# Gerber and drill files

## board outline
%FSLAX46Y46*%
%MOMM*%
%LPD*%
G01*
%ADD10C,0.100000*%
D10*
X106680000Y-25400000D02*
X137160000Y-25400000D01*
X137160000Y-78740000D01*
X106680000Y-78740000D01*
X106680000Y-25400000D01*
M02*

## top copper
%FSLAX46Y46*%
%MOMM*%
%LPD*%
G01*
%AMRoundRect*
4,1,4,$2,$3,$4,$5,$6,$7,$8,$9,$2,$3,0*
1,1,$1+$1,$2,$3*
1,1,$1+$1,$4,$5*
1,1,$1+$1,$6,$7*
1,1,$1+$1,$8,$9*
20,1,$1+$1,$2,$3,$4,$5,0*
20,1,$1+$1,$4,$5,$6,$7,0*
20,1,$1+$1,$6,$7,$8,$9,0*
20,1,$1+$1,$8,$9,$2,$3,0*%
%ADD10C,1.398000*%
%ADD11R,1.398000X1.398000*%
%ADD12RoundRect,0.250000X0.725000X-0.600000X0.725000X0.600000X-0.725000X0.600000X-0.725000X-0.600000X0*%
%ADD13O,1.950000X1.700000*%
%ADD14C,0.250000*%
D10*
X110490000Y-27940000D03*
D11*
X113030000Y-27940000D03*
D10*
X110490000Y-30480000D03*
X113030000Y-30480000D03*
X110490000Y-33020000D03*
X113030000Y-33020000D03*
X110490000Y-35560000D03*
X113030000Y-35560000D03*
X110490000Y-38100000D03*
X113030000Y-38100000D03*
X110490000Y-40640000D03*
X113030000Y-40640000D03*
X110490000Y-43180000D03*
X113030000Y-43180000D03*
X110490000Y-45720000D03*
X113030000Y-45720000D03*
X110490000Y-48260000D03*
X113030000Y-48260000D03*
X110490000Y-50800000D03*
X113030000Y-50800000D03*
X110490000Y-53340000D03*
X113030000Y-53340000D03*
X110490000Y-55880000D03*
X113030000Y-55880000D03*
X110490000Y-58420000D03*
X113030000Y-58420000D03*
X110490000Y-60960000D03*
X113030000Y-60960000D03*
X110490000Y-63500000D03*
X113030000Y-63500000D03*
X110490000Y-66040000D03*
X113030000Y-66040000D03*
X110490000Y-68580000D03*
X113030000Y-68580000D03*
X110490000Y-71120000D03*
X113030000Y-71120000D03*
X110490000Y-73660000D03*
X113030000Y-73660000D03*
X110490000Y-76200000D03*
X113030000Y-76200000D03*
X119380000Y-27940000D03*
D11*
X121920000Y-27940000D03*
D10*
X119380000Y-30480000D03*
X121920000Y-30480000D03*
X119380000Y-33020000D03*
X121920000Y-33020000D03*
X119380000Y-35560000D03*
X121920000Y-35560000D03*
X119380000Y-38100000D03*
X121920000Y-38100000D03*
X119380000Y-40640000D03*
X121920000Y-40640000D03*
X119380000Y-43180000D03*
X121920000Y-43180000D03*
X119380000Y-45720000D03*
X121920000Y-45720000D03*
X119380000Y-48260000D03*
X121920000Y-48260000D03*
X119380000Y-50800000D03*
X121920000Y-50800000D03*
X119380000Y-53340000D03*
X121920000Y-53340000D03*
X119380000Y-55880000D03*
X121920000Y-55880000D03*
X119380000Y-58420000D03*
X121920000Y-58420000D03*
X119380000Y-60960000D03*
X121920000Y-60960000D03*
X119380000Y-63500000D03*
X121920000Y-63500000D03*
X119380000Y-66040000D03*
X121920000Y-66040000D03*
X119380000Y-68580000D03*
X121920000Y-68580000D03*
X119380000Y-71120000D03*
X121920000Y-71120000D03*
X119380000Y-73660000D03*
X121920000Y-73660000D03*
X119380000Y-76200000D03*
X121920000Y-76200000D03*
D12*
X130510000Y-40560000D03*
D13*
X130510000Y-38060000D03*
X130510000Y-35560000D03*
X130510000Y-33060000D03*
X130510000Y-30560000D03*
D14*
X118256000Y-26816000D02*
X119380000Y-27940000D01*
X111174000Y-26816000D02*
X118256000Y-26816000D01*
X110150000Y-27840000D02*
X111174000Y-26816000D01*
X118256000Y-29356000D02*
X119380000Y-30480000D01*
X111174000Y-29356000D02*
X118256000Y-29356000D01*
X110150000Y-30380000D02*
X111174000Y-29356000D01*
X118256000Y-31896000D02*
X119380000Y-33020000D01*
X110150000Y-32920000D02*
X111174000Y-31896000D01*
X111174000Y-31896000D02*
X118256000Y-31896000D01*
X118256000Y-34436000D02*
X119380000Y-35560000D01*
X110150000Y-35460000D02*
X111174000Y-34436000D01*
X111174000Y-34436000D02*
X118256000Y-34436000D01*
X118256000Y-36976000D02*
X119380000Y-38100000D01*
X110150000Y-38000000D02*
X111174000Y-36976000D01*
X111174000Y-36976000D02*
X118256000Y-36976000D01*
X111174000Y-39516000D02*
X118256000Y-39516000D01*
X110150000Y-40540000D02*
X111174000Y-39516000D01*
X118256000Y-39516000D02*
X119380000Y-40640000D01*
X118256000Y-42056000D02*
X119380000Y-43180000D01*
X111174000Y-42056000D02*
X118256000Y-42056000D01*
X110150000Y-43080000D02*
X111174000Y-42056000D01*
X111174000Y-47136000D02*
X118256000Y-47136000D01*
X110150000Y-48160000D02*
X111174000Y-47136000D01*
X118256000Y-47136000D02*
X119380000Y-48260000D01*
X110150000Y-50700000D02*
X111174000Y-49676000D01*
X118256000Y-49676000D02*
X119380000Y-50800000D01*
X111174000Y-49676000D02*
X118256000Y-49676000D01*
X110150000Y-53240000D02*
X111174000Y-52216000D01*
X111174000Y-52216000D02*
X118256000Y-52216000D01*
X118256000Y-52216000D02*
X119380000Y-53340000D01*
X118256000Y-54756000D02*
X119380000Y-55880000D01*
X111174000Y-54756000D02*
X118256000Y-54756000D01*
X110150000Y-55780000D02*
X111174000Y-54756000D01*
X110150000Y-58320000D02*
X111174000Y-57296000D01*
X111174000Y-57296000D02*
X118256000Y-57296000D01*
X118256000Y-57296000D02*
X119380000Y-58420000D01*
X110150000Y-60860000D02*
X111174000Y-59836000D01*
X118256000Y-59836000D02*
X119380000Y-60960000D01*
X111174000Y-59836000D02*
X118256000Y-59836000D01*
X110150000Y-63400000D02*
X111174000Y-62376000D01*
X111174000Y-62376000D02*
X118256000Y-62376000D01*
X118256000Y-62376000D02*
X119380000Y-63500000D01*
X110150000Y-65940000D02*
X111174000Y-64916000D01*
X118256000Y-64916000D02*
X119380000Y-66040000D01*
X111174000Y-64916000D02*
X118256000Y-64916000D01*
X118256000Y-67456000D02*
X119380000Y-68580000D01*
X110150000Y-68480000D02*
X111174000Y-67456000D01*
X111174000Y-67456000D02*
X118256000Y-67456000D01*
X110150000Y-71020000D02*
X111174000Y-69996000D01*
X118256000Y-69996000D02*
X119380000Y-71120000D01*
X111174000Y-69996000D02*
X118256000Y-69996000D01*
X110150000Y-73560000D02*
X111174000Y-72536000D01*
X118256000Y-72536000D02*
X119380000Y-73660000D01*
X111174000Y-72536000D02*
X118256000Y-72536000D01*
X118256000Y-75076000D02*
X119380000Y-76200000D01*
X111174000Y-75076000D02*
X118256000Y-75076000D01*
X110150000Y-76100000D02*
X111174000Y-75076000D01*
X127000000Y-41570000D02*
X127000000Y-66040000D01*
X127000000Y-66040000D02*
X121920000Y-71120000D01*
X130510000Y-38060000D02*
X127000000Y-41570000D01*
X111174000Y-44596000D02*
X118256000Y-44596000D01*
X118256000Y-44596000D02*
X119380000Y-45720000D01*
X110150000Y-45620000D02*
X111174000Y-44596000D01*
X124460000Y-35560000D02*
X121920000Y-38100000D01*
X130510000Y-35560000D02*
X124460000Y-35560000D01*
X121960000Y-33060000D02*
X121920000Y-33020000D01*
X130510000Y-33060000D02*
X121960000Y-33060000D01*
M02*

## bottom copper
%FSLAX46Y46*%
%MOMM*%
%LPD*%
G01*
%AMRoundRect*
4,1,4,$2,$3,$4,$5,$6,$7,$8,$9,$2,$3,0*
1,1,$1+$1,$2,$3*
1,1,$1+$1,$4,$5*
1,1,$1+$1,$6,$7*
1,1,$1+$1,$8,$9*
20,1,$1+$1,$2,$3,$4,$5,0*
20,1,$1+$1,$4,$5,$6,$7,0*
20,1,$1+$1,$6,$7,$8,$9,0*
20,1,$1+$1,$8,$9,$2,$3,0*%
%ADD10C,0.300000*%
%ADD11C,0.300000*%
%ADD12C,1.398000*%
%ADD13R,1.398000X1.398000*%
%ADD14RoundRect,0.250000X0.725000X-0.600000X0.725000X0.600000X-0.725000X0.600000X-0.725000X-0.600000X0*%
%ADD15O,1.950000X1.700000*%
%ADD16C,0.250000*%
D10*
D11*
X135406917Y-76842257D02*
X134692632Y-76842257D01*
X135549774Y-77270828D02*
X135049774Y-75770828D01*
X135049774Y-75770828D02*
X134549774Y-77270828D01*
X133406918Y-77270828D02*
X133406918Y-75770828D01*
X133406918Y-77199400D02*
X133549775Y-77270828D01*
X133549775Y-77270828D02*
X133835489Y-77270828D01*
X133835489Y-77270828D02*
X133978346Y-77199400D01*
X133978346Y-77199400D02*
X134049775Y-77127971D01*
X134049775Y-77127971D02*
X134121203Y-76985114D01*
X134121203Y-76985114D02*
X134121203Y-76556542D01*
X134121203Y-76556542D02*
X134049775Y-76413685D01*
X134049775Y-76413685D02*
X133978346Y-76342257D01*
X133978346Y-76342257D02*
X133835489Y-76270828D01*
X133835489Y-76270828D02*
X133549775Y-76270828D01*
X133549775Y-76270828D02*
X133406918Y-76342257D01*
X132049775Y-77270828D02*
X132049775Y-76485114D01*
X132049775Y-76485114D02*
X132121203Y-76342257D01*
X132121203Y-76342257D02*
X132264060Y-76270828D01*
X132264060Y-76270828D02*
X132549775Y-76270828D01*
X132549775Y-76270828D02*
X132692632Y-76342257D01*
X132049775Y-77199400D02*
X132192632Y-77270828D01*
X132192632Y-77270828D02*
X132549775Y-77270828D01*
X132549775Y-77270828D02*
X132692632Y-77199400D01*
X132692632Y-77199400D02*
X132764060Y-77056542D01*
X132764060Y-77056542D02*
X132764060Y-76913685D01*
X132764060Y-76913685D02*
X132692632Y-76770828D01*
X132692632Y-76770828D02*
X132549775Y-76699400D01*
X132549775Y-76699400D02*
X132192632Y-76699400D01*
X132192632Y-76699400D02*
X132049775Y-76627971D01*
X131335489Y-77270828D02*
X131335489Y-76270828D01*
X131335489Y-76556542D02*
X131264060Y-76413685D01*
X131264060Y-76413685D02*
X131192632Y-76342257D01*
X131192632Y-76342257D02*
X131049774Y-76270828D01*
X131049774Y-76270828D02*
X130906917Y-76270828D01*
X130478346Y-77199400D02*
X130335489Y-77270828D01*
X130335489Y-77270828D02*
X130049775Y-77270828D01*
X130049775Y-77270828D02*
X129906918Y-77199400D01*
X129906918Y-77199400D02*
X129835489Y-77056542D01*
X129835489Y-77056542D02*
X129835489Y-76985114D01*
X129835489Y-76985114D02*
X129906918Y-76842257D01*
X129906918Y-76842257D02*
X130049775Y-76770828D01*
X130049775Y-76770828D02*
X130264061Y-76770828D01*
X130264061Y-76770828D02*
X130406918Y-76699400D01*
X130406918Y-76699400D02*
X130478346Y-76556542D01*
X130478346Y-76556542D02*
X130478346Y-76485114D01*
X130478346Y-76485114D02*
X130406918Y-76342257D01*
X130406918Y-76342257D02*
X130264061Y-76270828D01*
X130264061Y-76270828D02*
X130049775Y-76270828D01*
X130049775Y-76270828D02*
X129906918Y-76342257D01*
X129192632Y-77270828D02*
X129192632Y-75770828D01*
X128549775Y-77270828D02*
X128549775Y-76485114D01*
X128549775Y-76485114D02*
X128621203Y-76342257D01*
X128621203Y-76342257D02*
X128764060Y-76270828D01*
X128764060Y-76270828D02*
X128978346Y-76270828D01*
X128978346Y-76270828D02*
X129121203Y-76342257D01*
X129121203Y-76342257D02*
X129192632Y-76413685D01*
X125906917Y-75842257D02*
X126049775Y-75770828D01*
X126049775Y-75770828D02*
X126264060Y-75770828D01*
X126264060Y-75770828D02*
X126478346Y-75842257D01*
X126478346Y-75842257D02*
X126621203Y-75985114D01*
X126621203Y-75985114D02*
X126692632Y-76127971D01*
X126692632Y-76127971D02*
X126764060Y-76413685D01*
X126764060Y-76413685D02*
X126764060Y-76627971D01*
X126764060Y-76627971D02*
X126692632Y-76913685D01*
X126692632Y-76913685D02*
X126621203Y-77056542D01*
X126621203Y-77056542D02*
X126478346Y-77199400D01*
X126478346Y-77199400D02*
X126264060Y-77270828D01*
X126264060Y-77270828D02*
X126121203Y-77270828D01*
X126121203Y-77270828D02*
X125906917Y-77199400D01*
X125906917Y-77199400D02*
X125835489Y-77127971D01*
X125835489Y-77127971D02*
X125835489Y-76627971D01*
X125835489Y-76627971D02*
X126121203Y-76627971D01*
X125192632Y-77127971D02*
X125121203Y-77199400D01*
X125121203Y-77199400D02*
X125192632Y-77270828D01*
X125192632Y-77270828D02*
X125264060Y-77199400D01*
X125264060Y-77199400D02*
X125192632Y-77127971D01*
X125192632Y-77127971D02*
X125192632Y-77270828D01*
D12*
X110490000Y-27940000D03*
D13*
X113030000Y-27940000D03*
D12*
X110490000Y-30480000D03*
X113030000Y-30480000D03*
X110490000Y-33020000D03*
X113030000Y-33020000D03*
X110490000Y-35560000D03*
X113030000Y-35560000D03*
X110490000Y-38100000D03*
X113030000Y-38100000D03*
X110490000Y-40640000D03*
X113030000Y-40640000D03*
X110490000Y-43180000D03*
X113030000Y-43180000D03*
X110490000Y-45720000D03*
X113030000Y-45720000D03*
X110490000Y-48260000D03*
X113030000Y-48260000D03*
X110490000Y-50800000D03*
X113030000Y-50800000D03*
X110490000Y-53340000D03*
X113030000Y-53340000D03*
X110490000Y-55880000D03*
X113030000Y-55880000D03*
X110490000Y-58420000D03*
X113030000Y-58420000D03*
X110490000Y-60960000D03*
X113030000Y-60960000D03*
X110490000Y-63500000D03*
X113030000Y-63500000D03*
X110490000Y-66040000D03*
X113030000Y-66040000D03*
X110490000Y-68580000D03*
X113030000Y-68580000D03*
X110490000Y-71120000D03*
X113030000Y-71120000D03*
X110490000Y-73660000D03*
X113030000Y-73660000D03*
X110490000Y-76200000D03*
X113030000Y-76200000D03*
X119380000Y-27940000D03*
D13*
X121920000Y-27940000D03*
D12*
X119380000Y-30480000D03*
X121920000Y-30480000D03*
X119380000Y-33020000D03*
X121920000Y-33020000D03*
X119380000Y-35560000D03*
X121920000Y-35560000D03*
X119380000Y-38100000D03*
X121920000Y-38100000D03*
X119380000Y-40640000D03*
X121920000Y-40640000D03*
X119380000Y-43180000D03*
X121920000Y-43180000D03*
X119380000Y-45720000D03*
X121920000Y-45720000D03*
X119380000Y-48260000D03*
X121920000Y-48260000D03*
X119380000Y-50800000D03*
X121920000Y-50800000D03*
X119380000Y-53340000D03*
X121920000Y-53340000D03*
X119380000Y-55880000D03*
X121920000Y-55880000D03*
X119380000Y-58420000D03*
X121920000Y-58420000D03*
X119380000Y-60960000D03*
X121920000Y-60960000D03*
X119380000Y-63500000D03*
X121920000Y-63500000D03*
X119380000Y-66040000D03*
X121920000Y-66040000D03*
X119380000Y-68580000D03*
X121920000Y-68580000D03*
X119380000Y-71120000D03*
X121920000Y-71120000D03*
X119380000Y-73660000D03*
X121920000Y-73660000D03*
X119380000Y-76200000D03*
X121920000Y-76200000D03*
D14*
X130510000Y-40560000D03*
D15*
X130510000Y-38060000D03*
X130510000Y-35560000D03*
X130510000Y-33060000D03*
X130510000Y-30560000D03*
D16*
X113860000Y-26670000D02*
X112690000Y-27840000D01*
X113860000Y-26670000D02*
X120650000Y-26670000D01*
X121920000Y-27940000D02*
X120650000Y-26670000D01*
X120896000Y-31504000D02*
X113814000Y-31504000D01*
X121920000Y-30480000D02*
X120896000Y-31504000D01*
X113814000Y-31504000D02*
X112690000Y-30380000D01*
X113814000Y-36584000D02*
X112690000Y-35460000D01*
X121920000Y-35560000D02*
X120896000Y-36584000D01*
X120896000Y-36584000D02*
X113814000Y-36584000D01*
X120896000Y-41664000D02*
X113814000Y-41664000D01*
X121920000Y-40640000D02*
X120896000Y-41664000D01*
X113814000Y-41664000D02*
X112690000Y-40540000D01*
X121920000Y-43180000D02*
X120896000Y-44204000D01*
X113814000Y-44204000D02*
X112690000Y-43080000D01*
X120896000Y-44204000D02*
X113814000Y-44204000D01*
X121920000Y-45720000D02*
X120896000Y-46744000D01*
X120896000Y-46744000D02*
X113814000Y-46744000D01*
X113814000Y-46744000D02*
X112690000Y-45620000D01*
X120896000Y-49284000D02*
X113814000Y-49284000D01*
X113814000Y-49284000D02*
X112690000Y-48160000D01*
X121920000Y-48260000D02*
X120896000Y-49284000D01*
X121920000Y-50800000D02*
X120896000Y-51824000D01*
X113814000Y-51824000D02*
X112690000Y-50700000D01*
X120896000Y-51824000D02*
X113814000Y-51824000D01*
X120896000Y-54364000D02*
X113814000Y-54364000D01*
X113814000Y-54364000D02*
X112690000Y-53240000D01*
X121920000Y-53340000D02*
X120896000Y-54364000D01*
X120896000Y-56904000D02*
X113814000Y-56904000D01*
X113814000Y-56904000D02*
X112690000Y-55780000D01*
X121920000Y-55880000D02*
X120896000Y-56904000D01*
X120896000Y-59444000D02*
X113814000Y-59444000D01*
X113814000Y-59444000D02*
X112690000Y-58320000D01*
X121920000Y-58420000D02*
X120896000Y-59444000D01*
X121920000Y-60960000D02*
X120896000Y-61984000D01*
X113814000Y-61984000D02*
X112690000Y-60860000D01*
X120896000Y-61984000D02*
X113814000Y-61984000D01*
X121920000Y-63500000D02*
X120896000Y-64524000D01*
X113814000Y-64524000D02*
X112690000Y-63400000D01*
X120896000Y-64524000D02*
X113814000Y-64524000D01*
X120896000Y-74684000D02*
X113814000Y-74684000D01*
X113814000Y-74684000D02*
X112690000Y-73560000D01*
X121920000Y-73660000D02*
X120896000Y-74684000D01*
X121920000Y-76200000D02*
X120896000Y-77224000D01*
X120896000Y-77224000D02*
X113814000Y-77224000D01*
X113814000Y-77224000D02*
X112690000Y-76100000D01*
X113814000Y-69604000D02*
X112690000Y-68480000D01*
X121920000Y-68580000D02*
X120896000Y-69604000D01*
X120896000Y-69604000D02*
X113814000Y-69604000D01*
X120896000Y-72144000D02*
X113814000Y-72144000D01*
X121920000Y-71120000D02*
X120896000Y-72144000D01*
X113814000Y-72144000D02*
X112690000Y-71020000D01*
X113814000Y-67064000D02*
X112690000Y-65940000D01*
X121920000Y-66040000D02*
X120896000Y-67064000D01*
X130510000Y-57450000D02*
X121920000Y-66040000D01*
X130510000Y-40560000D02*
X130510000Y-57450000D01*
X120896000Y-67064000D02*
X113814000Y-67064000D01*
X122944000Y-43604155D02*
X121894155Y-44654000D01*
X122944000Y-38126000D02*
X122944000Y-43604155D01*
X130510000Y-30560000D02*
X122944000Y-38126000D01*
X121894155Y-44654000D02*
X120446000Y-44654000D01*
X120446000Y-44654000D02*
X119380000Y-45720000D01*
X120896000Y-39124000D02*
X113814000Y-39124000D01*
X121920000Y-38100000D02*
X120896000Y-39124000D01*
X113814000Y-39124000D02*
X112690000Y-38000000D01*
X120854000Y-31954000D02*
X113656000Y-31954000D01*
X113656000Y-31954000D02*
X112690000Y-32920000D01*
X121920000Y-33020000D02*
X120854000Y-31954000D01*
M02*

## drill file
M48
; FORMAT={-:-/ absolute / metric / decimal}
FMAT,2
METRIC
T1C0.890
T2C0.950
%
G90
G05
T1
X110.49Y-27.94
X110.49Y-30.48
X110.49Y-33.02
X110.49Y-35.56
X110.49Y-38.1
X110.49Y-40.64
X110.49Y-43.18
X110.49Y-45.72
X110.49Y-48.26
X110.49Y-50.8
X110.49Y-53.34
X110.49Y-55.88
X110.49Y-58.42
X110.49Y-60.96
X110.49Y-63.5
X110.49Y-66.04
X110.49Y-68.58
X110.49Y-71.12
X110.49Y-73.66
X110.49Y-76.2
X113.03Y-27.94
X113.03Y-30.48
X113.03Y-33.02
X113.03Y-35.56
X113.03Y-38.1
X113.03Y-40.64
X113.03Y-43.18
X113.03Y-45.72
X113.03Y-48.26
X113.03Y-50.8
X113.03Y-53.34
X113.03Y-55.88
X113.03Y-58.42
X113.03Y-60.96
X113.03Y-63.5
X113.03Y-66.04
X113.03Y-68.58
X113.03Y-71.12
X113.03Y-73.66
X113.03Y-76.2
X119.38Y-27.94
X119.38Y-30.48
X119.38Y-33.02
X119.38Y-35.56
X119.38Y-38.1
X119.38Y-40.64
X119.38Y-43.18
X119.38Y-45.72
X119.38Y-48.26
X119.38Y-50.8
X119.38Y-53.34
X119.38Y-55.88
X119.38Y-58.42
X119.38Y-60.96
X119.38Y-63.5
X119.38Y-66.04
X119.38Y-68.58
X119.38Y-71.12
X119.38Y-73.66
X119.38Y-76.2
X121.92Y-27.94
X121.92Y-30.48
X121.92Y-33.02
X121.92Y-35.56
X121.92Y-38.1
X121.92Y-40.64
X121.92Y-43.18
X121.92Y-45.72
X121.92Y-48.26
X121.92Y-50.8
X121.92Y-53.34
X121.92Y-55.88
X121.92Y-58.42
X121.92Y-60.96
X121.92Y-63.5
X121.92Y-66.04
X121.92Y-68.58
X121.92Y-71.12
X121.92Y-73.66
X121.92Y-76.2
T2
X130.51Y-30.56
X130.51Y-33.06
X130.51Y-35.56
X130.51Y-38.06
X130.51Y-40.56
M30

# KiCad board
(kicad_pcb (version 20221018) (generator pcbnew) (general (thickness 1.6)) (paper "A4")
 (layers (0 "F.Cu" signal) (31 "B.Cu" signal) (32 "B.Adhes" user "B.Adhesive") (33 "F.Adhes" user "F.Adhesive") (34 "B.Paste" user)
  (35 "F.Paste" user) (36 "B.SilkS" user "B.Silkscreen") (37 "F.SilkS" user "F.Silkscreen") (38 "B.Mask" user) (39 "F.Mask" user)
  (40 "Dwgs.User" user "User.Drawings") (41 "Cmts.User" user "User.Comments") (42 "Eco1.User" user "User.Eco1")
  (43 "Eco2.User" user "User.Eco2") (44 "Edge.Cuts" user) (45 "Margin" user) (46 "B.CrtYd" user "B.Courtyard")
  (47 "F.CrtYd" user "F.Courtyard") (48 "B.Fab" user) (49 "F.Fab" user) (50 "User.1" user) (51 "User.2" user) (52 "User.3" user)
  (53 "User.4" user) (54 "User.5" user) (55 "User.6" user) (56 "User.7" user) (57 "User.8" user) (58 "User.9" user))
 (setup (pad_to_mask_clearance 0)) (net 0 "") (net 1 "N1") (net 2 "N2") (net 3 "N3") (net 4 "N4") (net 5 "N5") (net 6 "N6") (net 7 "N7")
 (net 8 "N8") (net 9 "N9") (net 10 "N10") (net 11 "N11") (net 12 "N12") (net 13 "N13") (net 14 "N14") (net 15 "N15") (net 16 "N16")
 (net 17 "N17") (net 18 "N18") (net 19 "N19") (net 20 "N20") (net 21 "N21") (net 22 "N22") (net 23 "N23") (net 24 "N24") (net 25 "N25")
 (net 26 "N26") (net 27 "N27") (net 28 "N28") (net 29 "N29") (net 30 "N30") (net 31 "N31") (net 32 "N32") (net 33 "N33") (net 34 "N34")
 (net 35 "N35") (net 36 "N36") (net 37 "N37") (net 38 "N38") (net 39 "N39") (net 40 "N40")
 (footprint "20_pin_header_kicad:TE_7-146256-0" (layer "F.Cu") (at 111.76 52.07 -90)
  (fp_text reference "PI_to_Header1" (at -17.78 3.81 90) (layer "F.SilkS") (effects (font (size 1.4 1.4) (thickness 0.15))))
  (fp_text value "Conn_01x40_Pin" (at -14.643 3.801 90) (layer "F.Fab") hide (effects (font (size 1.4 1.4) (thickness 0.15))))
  (pad "1" thru_hole circle (at -24.13 1.27 270) (size 1.398 1.398) (drill 0.89) (layers "*.Cu" "*.Mask") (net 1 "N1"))
  (pad "2" thru_hole rect (at -24.13 -1.27 270) (size 1.398 1.398) (drill 0.89) (layers "*.Cu" "*.Mask") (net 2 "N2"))
  (pad "3" thru_hole circle (at -21.59 1.27 270) (size 1.398 1.398) (drill 0.89) (layers "*.Cu" "*.Mask") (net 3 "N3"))
  (pad "4" thru_hole circle (at -21.59 -1.27 270) (size 1.398 1.398) (drill 0.89) (layers "*.Cu" "*.Mask") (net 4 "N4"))
  (pad "5" thru_hole circle (at -19.05 1.27 270) (size 1.398 1.398) (drill 0.89) (layers "*.Cu" "*.Mask") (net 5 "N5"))
  (pad "6" thru_hole circle (at -19.05 -1.27 270) (size 1.398 1.398) (drill 0.89) (layers "*.Cu" "*.Mask") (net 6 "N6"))
  (pad "7" thru_hole circle (at -16.51 1.27 270) (size 1.398 1.398) (drill 0.89) (layers "*.Cu" "*.Mask") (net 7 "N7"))
  (pad "8" thru_hole circle (at -16.51 -1.27 270) (size 1.398 1.398) (drill 0.89) (layers "*.Cu" "*.Mask") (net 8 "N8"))
  (pad "9" thru_hole circle (at -13.97 1.27 270) (size 1.398 1.398) (drill 0.89) (layers "*.Cu" "*.Mask") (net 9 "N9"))
  (pad "10" thru_hole circle (at -13.97 -1.27 270) (size 1.398 1.398) (drill 0.89) (layers "*.Cu" "*.Mask") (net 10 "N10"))
  (pad "11" thru_hole circle (at -11.43 1.27 270) (size 1.398 1.398) (drill 0.89) (layers "*.Cu" "*.Mask") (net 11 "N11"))
  (pad "12" thru_hole circle (at -11.43 -1.27 270) (size 1.398 1.398) (drill 0.89) (layers "*.Cu" "*.Mask") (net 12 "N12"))
  (pad "13" thru_hole circle (at -8.89 1.27 270) (size 1.398 1.398) (drill 0.89) (layers "*.Cu" "*.Mask") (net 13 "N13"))
  (pad "14" thru_hole circle (at -8.89 -1.27 270) (size 1.398 1.398) (drill 0.89) (layers "*.Cu" "*.Mask") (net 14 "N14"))
  (pad "15" thru_hole circle (at -6.35 1.27 270) (size 1.398 1.398) (drill 0.89) (layers "*.Cu" "*.Mask") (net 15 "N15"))
  (pad "16" thru_hole circle (at -6.35 -1.27 270) (size 1.398 1.398) (drill 0.89) (layers "*.Cu" "*.Mask") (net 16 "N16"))
  (pad "17" thru_hole circle (at -3.81 1.27 270) (size 1.398 1.398) (drill 0.89) (layers "*.Cu" "*.Mask") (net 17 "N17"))
  (pad "18" thru_hole circle (at -3.81 -1.27 270) (size 1.398 1.398) (drill 0.89) (layers "*.Cu" "*.Mask") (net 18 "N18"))
  (pad "19" thru_hole circle (at -1.27 1.27 270) (size 1.398 1.398) (drill 0.89) (layers "*.Cu" "*.Mask") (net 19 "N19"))
  (pad "20" thru_hole circle (at -1.27 -1.27 270) (size 1.398 1.398) (drill 0.89) (layers "*.Cu" "*.Mask") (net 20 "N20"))
  (pad "21" thru_hole circle (at 1.27 1.27 270) (size 1.398 1.398) (drill 0.89) (layers "*.Cu" "*.Mask") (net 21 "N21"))
  (pad "22" thru_hole circle (at 1.27 -1.27 270) (size 1.398 1.398) (drill 0.89) (layers "*.Cu" "*.Mask") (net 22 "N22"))
  (pad "23" thru_hole circle (at 3.81 1.27 270) (size 1.398 1.398) (drill 0.89) (layers "*.Cu" "*.Mask") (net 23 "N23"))
  (pad "24" thru_hole circle (at 3.81 -1.27 270) (size 1.398 1.398) (drill 0.89) (layers "*.Cu" "*.Mask") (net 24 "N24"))
  (pad "25" thru_hole circle (at 6.35 1.27 270) (size 1.398 1.398) (drill 0.89) (layers "*.Cu" "*.Mask") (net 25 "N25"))
  (pad "26" thru_hole circle (at 6.35 -1.27 270) (size 1.398 1.398) (drill 0.89) (layers "*.Cu" "*.Mask") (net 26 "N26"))
  (pad "27" thru_hole circle (at 8.89 1.27 270) (size 1.398 1.398) (drill 0.89) (layers "*.Cu" "*.Mask") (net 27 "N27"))
  (pad "28" thru_hole circle (at 8.89 -1.27 270) (size 1.398 1.398) (drill 0.89) (layers "*.Cu" "*.Mask") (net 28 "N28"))
  (pad "29" thru_hole circle (at 11.43 1.27 270) (size 1.398 1.398) (drill 0.89) (layers "*.Cu" "*.Mask") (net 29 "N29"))
  (pad "30" thru_hole circle (at 11.43 -1.27 270) (size 1.398 1.398) (drill 0.89) (layers "*.Cu" "*.Mask") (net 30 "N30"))
  (pad "31" thru_hole circle (at 13.97 1.27 270) (size 1.398 1.398) (drill 0.89) (layers "*.Cu" "*.Mask") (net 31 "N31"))
  (pad "32" thru_hole circle (at 13.97 -1.27 270) (size 1.398 1.398) (drill 0.89) (layers "*.Cu" "*.Mask") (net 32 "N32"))
  (pad "33" thru_hole circle (at 16.51 1.27 270) (size 1.398 1.398) (drill 0.89) (layers "*.Cu" "*.Mask") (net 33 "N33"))
  (pad "34" thru_hole circle (at 16.51 -1.27 270) (size 1.398 1.398) (drill 0.89) (layers "*.Cu" "*.Mask") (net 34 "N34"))
  (pad "35" thru_hole circle (at 19.05 1.27 270) (size 1.398 1.398) (drill 0.89) (layers "*.Cu" "*.Mask") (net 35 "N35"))
  (pad "36" thru_hole circle (at 19.05 -1.27 270) (size 1.398 1.398) (drill 0.89) (layers "*.Cu" "*.Mask") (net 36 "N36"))
  (pad "37" thru_hole circle (at 21.59 1.27 270) (size 1.398 1.398) (drill 0.89) (layers "*.Cu" "*.Mask") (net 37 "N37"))
  (pad "38" thru_hole circle (at 21.59 -1.27 270) (size 1.398 1.398) (drill 0.89) (layers "*.Cu" "*.Mask") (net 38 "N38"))
  (pad "39" thru_hole circle (at 24.13 1.27 270) (size 1.398 1.398) (drill 0.89) (layers "*.Cu" "*.Mask") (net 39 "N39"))
  (pad "40" thru_hole circle (at 24.13 -1.27 270) (size 1.398 1.398) (drill 0.89) (layers "*.Cu" "*.Mask") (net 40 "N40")))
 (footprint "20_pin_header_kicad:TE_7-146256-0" (layer "F.Cu") (at 120.65 52.07 -90)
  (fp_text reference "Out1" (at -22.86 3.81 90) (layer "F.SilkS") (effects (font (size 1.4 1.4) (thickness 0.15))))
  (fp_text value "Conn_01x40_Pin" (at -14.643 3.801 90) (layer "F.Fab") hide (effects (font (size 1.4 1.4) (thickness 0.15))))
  (pad "1" thru_hole circle (at -24.13 1.27 270) (size 1.398 1.398) (drill 0.89) (layers "*.Cu" "*.Mask") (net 1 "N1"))
  (pad "2" thru_hole rect (at -24.13 -1.27 270) (size 1.398 1.398) (drill 0.89) (layers "*.Cu" "*.Mask") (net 2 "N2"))
  (pad "3" thru_hole circle (at -21.59 1.27 270) (size 1.398 1.398) (drill 0.89) (layers "*.Cu" "*.Mask") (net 3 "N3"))
  (pad "4" thru_hole circle (at -21.59 -1.27 270) (size 1.398 1.398) (drill 0.89) (layers "*.Cu" "*.Mask") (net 4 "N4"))
  (pad "5" thru_hole circle (at -19.05 1.27 270) (size 1.398 1.398) (drill 0.89) (layers "*.Cu" "*.Mask") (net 5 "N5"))
  (pad "6" thru_hole circle (at -19.05 -1.27 270) (size 1.398 1.398) (drill 0.89) (layers "*.Cu" "*.Mask") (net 6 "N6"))
  (pad "7" thru_hole circle (at -16.51 1.27 270) (size 1.398 1.398) (drill 0.89) (layers "*.Cu" "*.Mask") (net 7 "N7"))
  (pad "8" thru_hole circle (at -16.51 -1.27 270) (size 1.398 1.398) (drill 0.89) (layers "*.Cu" "*.Mask") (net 8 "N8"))
  (pad "9" thru_hole circle (at -13.97 1.27 270) (size 1.398 1.398) (drill 0.89) (layers "*.Cu" "*.Mask") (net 9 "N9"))
  (pad "10" thru_hole circle (at -13.97 -1.27 270) (size 1.398 1.398) (drill 0.89) (layers "*.Cu" "*.Mask") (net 10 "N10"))
  (pad "11" thru_hole circle (at -11.43 1.27 270) (size 1.398 1.398) (drill 0.89) (layers "*.Cu" "*.Mask") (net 11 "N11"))
  (pad "12" thru_hole circle (at -11.43 -1.27 270) (size 1.398 1.398) (drill 0.89) (layers "*.Cu" "*.Mask") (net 12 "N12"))
  (pad "13" thru_hole circle (at -8.89 1.27 270) (size 1.398 1.398) (drill 0.89) (layers "*.Cu" "*.Mask") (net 13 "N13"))
  (pad "14" thru_hole circle (at -8.89 -1.27 270) (size 1.398 1.398) (drill 0.89) (layers "*.Cu" "*.Mask") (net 14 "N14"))
  (pad "15" thru_hole circle (at -6.35 1.27 270) (size 1.398 1.398) (drill 0.89) (layers "*.Cu" "*.Mask") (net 15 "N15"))
  (pad "16" thru_hole circle (at -6.35 -1.27 270) (size 1.398 1.398) (drill 0.89) (layers "*.Cu" "*.Mask") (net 16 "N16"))
  (pad "17" thru_hole circle (at -3.81 1.27 270) (size 1.398 1.398) (drill 0.89) (layers "*.Cu" "*.Mask") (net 17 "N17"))
  (pad "18" thru_hole circle (at -3.81 -1.27 270) (size 1.398 1.398) (drill 0.89) (layers "*.Cu" "*.Mask") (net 18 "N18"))
  (pad "19" thru_hole circle (at -1.27 1.27 270) (size 1.398 1.398) (drill 0.89) (layers "*.Cu" "*.Mask") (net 19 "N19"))
  (pad "20" thru_hole circle (at -1.27 -1.27 270) (size 1.398 1.398) (drill 0.89) (layers "*.Cu" "*.Mask") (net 20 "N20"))
  (pad "21" thru_hole circle (at 1.27 1.27 270) (size 1.398 1.398) (drill 0.89) (layers "*.Cu" "*.Mask") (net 21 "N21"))
  (pad "22" thru_hole circle (at 1.27 -1.27 270) (size 1.398 1.398) (drill 0.89) (layers "*.Cu" "*.Mask") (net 22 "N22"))
  (pad "23" thru_hole circle (at 3.81 1.27 270) (size 1.398 1.398) (drill 0.89) (layers "*.Cu" "*.Mask") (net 23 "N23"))
  (pad "24" thru_hole circle (at 3.81 -1.27 270) (size 1.398 1.398) (drill 0.89) (layers "*.Cu" "*.Mask") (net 24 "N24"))
  (pad "25" thru_hole circle (at 6.35 1.27 270) (size 1.398 1.398) (drill 0.89) (layers "*.Cu" "*.Mask") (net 25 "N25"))
  (pad "26" thru_hole circle (at 6.35 -1.27 270) (size 1.398 1.398) (drill 0.89) (layers "*.Cu" "*.Mask") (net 26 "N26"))
  (pad "27" thru_hole circle (at 8.89 1.27 270) (size 1.398 1.398) (drill 0.89) (layers "*.Cu" "*.Mask") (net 27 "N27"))
  (pad "28" thru_hole circle (at 8.89 -1.27 270) (size 1.398 1.398) (drill 0.89) (layers "*.Cu" "*.Mask") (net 28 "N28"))
  (pad "29" thru_hole circle (at 11.43 1.27 270) (size 1.398 1.398) (drill 0.89) (layers "*.Cu" "*.Mask") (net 29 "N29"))
  (pad "30" thru_hole circle (at 11.43 -1.27 270) (size 1.398 1.398) (drill 0.89) (layers "*.Cu" "*.Mask") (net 30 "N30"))
  (pad "31" thru_hole circle (at 13.97 1.27 270) (size 1.398 1.398) (drill 0.89) (layers "*.Cu" "*.Mask") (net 31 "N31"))
  (pad "32" thru_hole circle (at 13.97 -1.27 270) (size 1.398 1.398) (drill 0.89) (layers "*.Cu" "*.Mask") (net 32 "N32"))
  (pad "33" thru_hole circle (at 16.51 1.27 270) (size 1.398 1.398) (drill 0.89) (layers "*.Cu" "*.Mask") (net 33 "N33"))
  (pad "34" thru_hole circle (at 16.51 -1.27 270) (size 1.398 1.398) (drill 0.89) (layers "*.Cu" "*.Mask") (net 34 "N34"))
  (pad "35" thru_hole circle (at 19.05 1.27 270) (size 1.398 1.398) (drill 0.89) (layers "*.Cu" "*.Mask") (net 35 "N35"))
  (pad "36" thru_hole circle (at 19.05 -1.27 270) (size 1.398 1.398) (drill 0.89) (layers "*.Cu" "*.Mask") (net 36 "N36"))
  (pad "37" thru_hole circle (at 21.59 1.27 270) (size 1.398 1.398) (drill 0.89) (layers "*.Cu" "*.Mask") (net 37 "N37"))
  (pad "38" thru_hole circle (at 21.59 -1.27 270) (size 1.398 1.398) (drill 0.89) (layers "*.Cu" "*.Mask") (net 38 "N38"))
  (pad "39" thru_hole circle (at 24.13 1.27 270) (size 1.398 1.398) (drill 0.89) (layers "*.Cu" "*.Mask") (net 39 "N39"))
  (pad "40" thru_hole circle (at 24.13 -1.27 270) (size 1.398 1.398) (drill 0.89) (layers "*.Cu" "*.Mask") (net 40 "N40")))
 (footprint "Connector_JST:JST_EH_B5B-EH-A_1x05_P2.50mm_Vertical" (layer "F.Cu") (at 130.51 40.56 90)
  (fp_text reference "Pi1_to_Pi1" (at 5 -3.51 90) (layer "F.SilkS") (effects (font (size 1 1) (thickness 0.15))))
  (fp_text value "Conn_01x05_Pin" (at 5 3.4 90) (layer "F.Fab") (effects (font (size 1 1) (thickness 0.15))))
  (pad "1" thru_hole roundrect (at 0 0 90) (size 1.7 1.95) (drill 0.95) (layers "*.Cu" "*.Mask") (roundrect_rratio 0.1470588235)
   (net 32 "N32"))
  (pad "2" thru_hole oval (at 2.5 0 90) (size 1.7 1.95) (drill 0.95) (layers "*.Cu" "*.Mask") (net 36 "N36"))
  (pad "3" thru_hole oval (at 5 0 90) (size 1.7 1.95) (drill 0.95) (layers "*.Cu" "*.Mask") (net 10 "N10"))
  (pad "4" thru_hole oval (at 7.5 0 90) (size 1.7 1.95) (drill 0.95) (layers "*.Cu" "*.Mask") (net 6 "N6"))
  (pad "5" thru_hole oval (at 10 0 90) (size 1.7 1.95) (drill 0.95) (layers "*.Cu" "*.Mask") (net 15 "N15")))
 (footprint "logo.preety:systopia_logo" (layer "F.Cu") (at 130.81 68.58)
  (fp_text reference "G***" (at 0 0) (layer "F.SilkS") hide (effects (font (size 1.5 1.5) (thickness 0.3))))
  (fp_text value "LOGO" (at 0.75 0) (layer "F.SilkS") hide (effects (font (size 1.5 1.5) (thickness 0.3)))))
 (gr_rect (start 106.68 25.4) (end 137.16 78.74) (stroke (width 0.1) (type default)) (fill none) (layer "Edge.Cuts"))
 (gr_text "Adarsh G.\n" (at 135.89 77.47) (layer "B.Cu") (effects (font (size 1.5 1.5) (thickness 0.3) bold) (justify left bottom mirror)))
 (segment (start 118.256 26.816) (end 119.38 27.94) (width 0.25) (layer "F.Cu") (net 1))
 (segment (start 111.174 26.816) (end 118.256 26.816) (width 0.25) (layer "F.Cu") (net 1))
 (segment (start 110.15 27.84) (end 111.174 26.816) (width 0.25) (layer "F.Cu") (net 1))
 (segment (start 113.86 26.67) (end 112.69 27.84) (width 0.25) (layer "B.Cu") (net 2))
 (segment (start 113.86 26.67) (end 120.65 26.67) (width 0.25) (layer "B.Cu") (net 2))
 (segment (start 121.92 27.94) (end 120.65 26.67) (width 0.25) (layer "B.Cu") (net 2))
 (segment (start 118.256 29.356) (end 119.38 30.48) (width 0.25) (layer "F.Cu") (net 3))
 (segment (start 111.174 29.356) (end 118.256 29.356) (width 0.25) (layer "F.Cu") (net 3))
 (segment (start 110.15 30.38) (end 111.174 29.356) (width 0.25) (layer "F.Cu") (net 3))
 (segment (start 120.896 31.504) (end 113.814 31.504) (width 0.25) (layer "B.Cu") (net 4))
 (segment (start 121.92 30.48) (end 120.896 31.504) (width 0.25) (layer "B.Cu") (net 4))
 (segment (start 113.814 31.504) (end 112.69 30.38) (width 0.25) (layer "B.Cu") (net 4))
 (segment (start 118.256 31.896) (end 119.38 33.02) (width 0.25) (layer "F.Cu") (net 5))
 (segment (start 110.15 32.92) (end 111.174 31.896) (width 0.25) (layer "F.Cu") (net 5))
 (segment (start 111.174 31.896) (end 118.256 31.896) (width 0.25) (layer "F.Cu") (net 5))
 (segment (start 118.256 34.436) (end 119.38 35.56) (width 0.25) (layer "F.Cu") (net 7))
 (segment (start 110.15 35.46) (end 111.174 34.436) (width 0.25) (layer "F.Cu") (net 7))
 (segment (start 111.174 34.436) (end 118.256 34.436) (width 0.25) (layer "F.Cu") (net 7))
 (segment (start 113.814 36.584) (end 112.69 35.46) (width 0.25) (layer "B.Cu") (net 8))
 (segment (start 121.92 35.56) (end 120.896 36.584) (width 0.25) (layer "B.Cu") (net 8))
 (segment (start 120.896 36.584) (end 113.814 36.584) (width 0.25) (layer "B.Cu") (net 8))
 (segment (start 118.256 36.976) (end 119.38 38.1) (width 0.25) (layer "F.Cu") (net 9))
 (segment (start 110.15 38) (end 111.174 36.976) (width 0.25) (layer "F.Cu") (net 9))
 (segment (start 111.174 36.976) (end 118.256 36.976) (width 0.25) (layer "F.Cu") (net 9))
 (segment (start 111.174 39.516) (end 118.256 39.516) (width 0.25) (layer "F.Cu") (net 11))
 (segment (start 110.15 40.54) (end 111.174 39.516) (width 0.25) (layer "F.Cu") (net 11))
 (segment (start 118.256 39.516) (end 119.38 40.64) (width 0.25) (layer "F.Cu") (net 11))
 (segment (start 120.896 41.664) (end 113.814 41.664) (width 0.25) (layer "B.Cu") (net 12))
 (segment (start 121.92 40.64) (end 120.896 41.664) (width 0.25) (layer "B.Cu") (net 12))
 (segment (start 113.814 41.664) (end 112.69 40.54) (width 0.25) (layer "B.Cu") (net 12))
 (segment (start 118.256 42.056) (end 119.38 43.18) (width 0.25) (layer "F.Cu") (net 13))
 (segment (start 111.174 42.056) (end 118.256 42.056) (width 0.25) (layer "F.Cu") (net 13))
 (segment (start 110.15 43.08) (end 111.174 42.056) (width 0.25) (layer "F.Cu") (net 13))
 (segment (start 121.92 43.18) (end 120.896 44.204) (width 0.25) (layer "B.Cu") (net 14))
 (segment (start 113.814 44.204) (end 112.69 43.08) (width 0.25) (layer "B.Cu") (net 14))
 (segment (start 120.896 44.204) (end 113.814 44.204) (width 0.25) (layer "B.Cu") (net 14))
 (segment (start 121.92 45.72) (end 120.896 46.744) (width 0.25) (layer "B.Cu") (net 16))
 (segment (start 120.896 46.744) (end 113.814 46.744) (width 0.25) (layer "B.Cu") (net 16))
 (segment (start 113.814 46.744) (end 112.69 45.62) (width 0.25) (layer "B.Cu") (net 16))
 (segment (start 111.174 47.136) (end 118.256 47.136) (width 0.25) (layer "F.Cu") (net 17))
 (segment (start 110.15 48.16) (end 111.174 47.136) (width 0.25) (layer "F.Cu") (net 17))
 (segment (start 118.256 47.136) (end 119.38 48.26) (width 0.25) (layer "F.Cu") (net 17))
 (segment (start 120.896 49.284) (end 113.814 49.284) (width 0.25) (layer "B.Cu") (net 18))
 (segment (start 113.814 49.284) (end 112.69 48.16) (width 0.25) (layer "B.Cu") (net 18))
 (segment (start 121.92 48.26) (end 120.896 49.284) (width 0.25) (layer "B.Cu") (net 18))
 (segment (start 110.15 50.7) (end 111.174 49.676) (width 0.25) (layer "F.Cu") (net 19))
 (segment (start 118.256 49.676) (end 119.38 50.8) (width 0.25) (layer "F.Cu") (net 19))
 (segment (start 111.174 49.676) (end 118.256 49.676) (width 0.25) (layer "F.Cu") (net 19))
 (segment (start 121.92 50.8) (end 120.896 51.824) (width 0.25) (layer "B.Cu") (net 20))
 (segment (start 113.814 51.824) (end 112.69 50.7) (width 0.25) (layer "B.Cu") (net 20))
 (segment (start 120.896 51.824) (end 113.814 51.824) (width 0.25) (layer "B.Cu") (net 20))
 (segment (start 110.15 53.24) (end 111.174 52.216) (width 0.25) (layer "F.Cu") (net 21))
 (segment (start 111.174 52.216) (end 118.256 52.216) (width 0.25) (layer "F.Cu") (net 21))
 (segment (start 118.256 52.216) (end 119.38 53.34) (width 0.25) (layer "F.Cu") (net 21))
 (segment (start 120.896 54.364) (end 113.814 54.364) (width 0.25) (layer "B.Cu") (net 22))
 (segment (start 113.814 54.364) (end 112.69 53.24) (width 0.25) (layer "B.Cu") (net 22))
 (segment (start 121.92 53.34) (end 120.896 54.364) (width 0.25) (layer "B.Cu") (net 22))
 (segment (start 118.256 54.756) (end 119.38 55.88) (width 0.25) (layer "F.Cu") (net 23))
 (segment (start 111.174 54.756) (end 118.256 54.756) (width 0.25) (layer "F.Cu") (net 23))
 (segment (start 110.15 55.78) (end 111.174 54.756) (width 0.25) (layer "F.Cu") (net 23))
 (segment (start 120.896 56.904) (end 113.814 56.904) (width 0.25) (layer "B.Cu") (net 24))
 (segment (start 113.814 56.904) (end 112.69 55.78) (width 0.25) (layer "B.Cu") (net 24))
 (segment (start 121.92 55.88) (end 120.896 56.904) (width 0.25) (layer "B.Cu") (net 24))
 (segment (start 110.15 58.32) (end 111.174 57.296) (width 0.25) (layer "F.Cu") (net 25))
 (segment (start 111.174 57.296) (end 118.256 57.296) (width 0.25) (layer "F.Cu") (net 25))
 (segment (start 118.256 57.296) (end 119.38 58.42) (width 0.25) (layer "F.Cu") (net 25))
 (segment (start 120.896 59.444) (end 113.814 59.444) (width 0.25) (layer "B.Cu") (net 26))
 (segment (start 113.814 59.444) (end 112.69 58.32) (width 0.25) (layer "B.Cu") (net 26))
 (segment (start 121.92 58.42) (end 120.896 59.444) (width 0.25) (layer "B.Cu") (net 26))
 (segment (start 110.15 60.86) (end 111.174 59.836) (width 0.25) (layer "F.Cu") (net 27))
 (segment (start 118.256 59.836) (end 119.38 60.96) (width 0.25) (layer "F.Cu") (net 27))
 (segment (start 111.174 59.836) (end 118.256 59.836) (width 0.25) (layer "F.Cu") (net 27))
 (segment (start 121.92 60.96) (end 120.896 61.984) (width 0.25) (layer "B.Cu") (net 28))
 (segment (start 113.814 61.984) (end 112.69 60.86) (width 0.25) (layer "B.Cu") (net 28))
 (segment (start 120.896 61.984) (end 113.814 61.984) (width 0.25) (layer "B.Cu") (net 28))
 (segment (start 110.15 63.4) (end 111.174 62.376) (width 0.25) (layer "F.Cu") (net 29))
 (segment (start 111.174 62.376) (end 118.256 62.376) (width 0.25) (layer "F.Cu") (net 29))
 (segment (start 118.256 62.376) (end 119.38 63.5) (width 0.25) (layer "F.Cu") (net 29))
 (segment (start 121.92 63.5) (end 120.896 64.524) (width 0.25) (layer "B.Cu") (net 30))
 (segment (start 113.814 64.524) (end 112.69 63.4) (width 0.25) (layer "B.Cu") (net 30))
 (segment (start 120.896 64.524) (end 113.814 64.524) (width 0.25) (layer "B.Cu") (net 30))
 (segment (start 110.15 65.94) (end 111.174 64.916) (width 0.25) (layer "F.Cu") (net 31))
 (segment (start 118.256 64.916) (end 119.38 66.04) (width 0.25) (layer "F.Cu") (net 31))
 (segment (start 111.174 64.916) (end 118.256 64.916) (width 0.25) (layer "F.Cu") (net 31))
 (segment (start 118.256 67.456) (end 119.38 68.58) (width 0.25) (layer "F.Cu") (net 33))
 (segment (start 110.15 68.48) (end 111.174 67.456) (width 0.25) (layer "F.Cu") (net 33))
 (segment (start 111.174 67.456) (end 118.256 67.456) (width 0.25) (layer "F.Cu") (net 33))
 (segment (start 110.15 71.02) (end 111.174 69.996) (width 0.25) (layer "F.Cu") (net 35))
 (segment (start 118.256 69.996) (end 119.38 71.12) (width 0.25) (layer "F.Cu") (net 35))
 (segment (start 111.174 69.996) (end 118.256 69.996) (width 0.25) (layer "F.Cu") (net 35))
 (segment (start 110.15 73.56) (end 111.174 72.536) (width 0.25) (layer "F.Cu") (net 37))
 (segment (start 118.256 72.536) (end 119.38 73.66) (width 0.25) (layer "F.Cu") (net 37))
 (segment (start 111.174 72.536) (end 118.256 72.536) (width 0.25) (layer "F.Cu") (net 37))
 (segment (start 120.896 74.684) (end 113.814 74.684) (width 0.25) (layer "B.Cu") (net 38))
 (segment (start 113.814 74.684) (end 112.69 73.56) (width 0.25) (layer "B.Cu") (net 38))
 (segment (start 121.92 73.66) (end 120.896 74.684) (width 0.25) (layer "B.Cu") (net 38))
 (segment (start 118.256 75.076) (end 119.38 76.2) (width 0.25) (layer "F.Cu") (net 39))
 (segment (start 111.174 75.076) (end 118.256 75.076) (width 0.25) (layer "F.Cu") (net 39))
 (segment (start 110.15 76.1) (end 111.174 75.076) (width 0.25) (layer "F.Cu") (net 39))
 (segment (start 121.92 76.2) (end 120.896 77.224) (width 0.25) (layer "B.Cu") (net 40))
 (segment (start 120.896 77.224) (end 113.814 77.224) (width 0.25) (layer "B.Cu") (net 40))
 (segment (start 113.814 77.224) (end 112.69 76.1) (width 0.25) (layer "B.Cu") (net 40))
 (segment (start 113.814 69.604) (end 112.69 68.48) (width 0.25) (layer "B.Cu") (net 34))
 (segment (start 121.92 68.58) (end 120.896 69.604) (width 0.25) (layer "B.Cu") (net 34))
 (segment (start 120.896 69.604) (end 113.814 69.604) (width 0.25) (layer "B.Cu") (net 34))
 (segment (start 127 41.57) (end 127 66.04) (width 0.25) (layer "F.Cu") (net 36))
 (segment (start 127 66.04) (end 121.92 71.12) (width 0.25) (layer "F.Cu") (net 36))
 (segment (start 130.51 38.06) (end 127 41.57) (width 0.25) (layer "F.Cu") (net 36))
 (segment (start 120.896 72.144) (end 113.814 72.144) (width 0.25) (layer "B.Cu") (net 36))
 (segment (start 121.92 71.12) (end 120.896 72.144) (width 0.25) (layer "B.Cu") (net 36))
 (segment (start 113.814 72.144) (end 112.69 71.02) (width 0.25) (layer "B.Cu") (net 36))
 (segment (start 113.814 67.064) (end 112.69 65.94) (width 0.25) (layer "B.Cu") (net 32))
 (segment (start 121.92 66.04) (end 120.896 67.064) (width 0.25) (layer "B.Cu") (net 32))
 (segment (start 130.51 57.45) (end 121.92 66.04) (width 0.25) (layer "B.Cu") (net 32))
 (segment (start 130.51 40.56) (end 130.51 57.45) (width 0.25) (layer "B.Cu") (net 32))
 (segment (start 120.896 67.064) (end 113.814 67.064) (width 0.25) (layer "B.Cu") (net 32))
 (segment (start 111.174 44.596) (end 118.256 44.596) (width 0.25) (layer "F.Cu") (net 15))
 (segment (start 118.256 44.596) (end 119.38 45.72) (width 0.25) (layer "F.Cu") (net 15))
 (segment (start 110.15 45.62) (end 111.174 44.596) (width 0.25) (layer "F.Cu") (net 15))
 (segment (start 122.944 43.604155) (end 121.894155 44.654) (width 0.25) (layer "B.Cu") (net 15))
 (segment (start 122.944 38.126) (end 122.944 43.604155) (width 0.25) (layer "B.Cu") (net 15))
 (segment (start 130.51 30.56) (end 122.944 38.126) (width 0.25) (layer "B.Cu") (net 15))
 (segment (start 121.894155 44.654) (end 120.446 44.654) (width 0.25) (layer "B.Cu") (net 15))
 (segment (start 120.446 44.654) (end 119.38 45.72) (width 0.25) (layer "B.Cu") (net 15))
 (segment (start 124.46 35.56) (end 121.92 38.1) (width 0.25) (layer "F.Cu") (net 10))
 (segment (start 130.51 35.56) (end 124.46 35.56) (width 0.25) (layer "F.Cu") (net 10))
 (segment (start 120.896 39.124) (end 113.814 39.124) (width 0.25) (layer "B.Cu") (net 10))
 (segment (start 121.92 38.1) (end 120.896 39.124) (width 0.25) (layer "B.Cu") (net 10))
 (segment (start 113.814 39.124) (end 112.69 38) (width 0.25) (layer "B.Cu") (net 10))
 (segment (start 121.96 33.06) (end 121.92 33.02) (width 0.25) (layer "F.Cu") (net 6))
 (segment (start 130.51 33.06) (end 121.96 33.06) (width 0.25) (layer "F.Cu") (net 6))
 (segment (start 120.854 31.954) (end 113.656 31.954) (width 0.25) (layer "B.Cu") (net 6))
 (segment (start 113.656 31.954) (end 112.69 32.92) (width 0.25) (layer "B.Cu") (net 6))
 (segment (start 121.92 33.02) (end 120.854 31.954) (width 0.25) (layer "B.Cu") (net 6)))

